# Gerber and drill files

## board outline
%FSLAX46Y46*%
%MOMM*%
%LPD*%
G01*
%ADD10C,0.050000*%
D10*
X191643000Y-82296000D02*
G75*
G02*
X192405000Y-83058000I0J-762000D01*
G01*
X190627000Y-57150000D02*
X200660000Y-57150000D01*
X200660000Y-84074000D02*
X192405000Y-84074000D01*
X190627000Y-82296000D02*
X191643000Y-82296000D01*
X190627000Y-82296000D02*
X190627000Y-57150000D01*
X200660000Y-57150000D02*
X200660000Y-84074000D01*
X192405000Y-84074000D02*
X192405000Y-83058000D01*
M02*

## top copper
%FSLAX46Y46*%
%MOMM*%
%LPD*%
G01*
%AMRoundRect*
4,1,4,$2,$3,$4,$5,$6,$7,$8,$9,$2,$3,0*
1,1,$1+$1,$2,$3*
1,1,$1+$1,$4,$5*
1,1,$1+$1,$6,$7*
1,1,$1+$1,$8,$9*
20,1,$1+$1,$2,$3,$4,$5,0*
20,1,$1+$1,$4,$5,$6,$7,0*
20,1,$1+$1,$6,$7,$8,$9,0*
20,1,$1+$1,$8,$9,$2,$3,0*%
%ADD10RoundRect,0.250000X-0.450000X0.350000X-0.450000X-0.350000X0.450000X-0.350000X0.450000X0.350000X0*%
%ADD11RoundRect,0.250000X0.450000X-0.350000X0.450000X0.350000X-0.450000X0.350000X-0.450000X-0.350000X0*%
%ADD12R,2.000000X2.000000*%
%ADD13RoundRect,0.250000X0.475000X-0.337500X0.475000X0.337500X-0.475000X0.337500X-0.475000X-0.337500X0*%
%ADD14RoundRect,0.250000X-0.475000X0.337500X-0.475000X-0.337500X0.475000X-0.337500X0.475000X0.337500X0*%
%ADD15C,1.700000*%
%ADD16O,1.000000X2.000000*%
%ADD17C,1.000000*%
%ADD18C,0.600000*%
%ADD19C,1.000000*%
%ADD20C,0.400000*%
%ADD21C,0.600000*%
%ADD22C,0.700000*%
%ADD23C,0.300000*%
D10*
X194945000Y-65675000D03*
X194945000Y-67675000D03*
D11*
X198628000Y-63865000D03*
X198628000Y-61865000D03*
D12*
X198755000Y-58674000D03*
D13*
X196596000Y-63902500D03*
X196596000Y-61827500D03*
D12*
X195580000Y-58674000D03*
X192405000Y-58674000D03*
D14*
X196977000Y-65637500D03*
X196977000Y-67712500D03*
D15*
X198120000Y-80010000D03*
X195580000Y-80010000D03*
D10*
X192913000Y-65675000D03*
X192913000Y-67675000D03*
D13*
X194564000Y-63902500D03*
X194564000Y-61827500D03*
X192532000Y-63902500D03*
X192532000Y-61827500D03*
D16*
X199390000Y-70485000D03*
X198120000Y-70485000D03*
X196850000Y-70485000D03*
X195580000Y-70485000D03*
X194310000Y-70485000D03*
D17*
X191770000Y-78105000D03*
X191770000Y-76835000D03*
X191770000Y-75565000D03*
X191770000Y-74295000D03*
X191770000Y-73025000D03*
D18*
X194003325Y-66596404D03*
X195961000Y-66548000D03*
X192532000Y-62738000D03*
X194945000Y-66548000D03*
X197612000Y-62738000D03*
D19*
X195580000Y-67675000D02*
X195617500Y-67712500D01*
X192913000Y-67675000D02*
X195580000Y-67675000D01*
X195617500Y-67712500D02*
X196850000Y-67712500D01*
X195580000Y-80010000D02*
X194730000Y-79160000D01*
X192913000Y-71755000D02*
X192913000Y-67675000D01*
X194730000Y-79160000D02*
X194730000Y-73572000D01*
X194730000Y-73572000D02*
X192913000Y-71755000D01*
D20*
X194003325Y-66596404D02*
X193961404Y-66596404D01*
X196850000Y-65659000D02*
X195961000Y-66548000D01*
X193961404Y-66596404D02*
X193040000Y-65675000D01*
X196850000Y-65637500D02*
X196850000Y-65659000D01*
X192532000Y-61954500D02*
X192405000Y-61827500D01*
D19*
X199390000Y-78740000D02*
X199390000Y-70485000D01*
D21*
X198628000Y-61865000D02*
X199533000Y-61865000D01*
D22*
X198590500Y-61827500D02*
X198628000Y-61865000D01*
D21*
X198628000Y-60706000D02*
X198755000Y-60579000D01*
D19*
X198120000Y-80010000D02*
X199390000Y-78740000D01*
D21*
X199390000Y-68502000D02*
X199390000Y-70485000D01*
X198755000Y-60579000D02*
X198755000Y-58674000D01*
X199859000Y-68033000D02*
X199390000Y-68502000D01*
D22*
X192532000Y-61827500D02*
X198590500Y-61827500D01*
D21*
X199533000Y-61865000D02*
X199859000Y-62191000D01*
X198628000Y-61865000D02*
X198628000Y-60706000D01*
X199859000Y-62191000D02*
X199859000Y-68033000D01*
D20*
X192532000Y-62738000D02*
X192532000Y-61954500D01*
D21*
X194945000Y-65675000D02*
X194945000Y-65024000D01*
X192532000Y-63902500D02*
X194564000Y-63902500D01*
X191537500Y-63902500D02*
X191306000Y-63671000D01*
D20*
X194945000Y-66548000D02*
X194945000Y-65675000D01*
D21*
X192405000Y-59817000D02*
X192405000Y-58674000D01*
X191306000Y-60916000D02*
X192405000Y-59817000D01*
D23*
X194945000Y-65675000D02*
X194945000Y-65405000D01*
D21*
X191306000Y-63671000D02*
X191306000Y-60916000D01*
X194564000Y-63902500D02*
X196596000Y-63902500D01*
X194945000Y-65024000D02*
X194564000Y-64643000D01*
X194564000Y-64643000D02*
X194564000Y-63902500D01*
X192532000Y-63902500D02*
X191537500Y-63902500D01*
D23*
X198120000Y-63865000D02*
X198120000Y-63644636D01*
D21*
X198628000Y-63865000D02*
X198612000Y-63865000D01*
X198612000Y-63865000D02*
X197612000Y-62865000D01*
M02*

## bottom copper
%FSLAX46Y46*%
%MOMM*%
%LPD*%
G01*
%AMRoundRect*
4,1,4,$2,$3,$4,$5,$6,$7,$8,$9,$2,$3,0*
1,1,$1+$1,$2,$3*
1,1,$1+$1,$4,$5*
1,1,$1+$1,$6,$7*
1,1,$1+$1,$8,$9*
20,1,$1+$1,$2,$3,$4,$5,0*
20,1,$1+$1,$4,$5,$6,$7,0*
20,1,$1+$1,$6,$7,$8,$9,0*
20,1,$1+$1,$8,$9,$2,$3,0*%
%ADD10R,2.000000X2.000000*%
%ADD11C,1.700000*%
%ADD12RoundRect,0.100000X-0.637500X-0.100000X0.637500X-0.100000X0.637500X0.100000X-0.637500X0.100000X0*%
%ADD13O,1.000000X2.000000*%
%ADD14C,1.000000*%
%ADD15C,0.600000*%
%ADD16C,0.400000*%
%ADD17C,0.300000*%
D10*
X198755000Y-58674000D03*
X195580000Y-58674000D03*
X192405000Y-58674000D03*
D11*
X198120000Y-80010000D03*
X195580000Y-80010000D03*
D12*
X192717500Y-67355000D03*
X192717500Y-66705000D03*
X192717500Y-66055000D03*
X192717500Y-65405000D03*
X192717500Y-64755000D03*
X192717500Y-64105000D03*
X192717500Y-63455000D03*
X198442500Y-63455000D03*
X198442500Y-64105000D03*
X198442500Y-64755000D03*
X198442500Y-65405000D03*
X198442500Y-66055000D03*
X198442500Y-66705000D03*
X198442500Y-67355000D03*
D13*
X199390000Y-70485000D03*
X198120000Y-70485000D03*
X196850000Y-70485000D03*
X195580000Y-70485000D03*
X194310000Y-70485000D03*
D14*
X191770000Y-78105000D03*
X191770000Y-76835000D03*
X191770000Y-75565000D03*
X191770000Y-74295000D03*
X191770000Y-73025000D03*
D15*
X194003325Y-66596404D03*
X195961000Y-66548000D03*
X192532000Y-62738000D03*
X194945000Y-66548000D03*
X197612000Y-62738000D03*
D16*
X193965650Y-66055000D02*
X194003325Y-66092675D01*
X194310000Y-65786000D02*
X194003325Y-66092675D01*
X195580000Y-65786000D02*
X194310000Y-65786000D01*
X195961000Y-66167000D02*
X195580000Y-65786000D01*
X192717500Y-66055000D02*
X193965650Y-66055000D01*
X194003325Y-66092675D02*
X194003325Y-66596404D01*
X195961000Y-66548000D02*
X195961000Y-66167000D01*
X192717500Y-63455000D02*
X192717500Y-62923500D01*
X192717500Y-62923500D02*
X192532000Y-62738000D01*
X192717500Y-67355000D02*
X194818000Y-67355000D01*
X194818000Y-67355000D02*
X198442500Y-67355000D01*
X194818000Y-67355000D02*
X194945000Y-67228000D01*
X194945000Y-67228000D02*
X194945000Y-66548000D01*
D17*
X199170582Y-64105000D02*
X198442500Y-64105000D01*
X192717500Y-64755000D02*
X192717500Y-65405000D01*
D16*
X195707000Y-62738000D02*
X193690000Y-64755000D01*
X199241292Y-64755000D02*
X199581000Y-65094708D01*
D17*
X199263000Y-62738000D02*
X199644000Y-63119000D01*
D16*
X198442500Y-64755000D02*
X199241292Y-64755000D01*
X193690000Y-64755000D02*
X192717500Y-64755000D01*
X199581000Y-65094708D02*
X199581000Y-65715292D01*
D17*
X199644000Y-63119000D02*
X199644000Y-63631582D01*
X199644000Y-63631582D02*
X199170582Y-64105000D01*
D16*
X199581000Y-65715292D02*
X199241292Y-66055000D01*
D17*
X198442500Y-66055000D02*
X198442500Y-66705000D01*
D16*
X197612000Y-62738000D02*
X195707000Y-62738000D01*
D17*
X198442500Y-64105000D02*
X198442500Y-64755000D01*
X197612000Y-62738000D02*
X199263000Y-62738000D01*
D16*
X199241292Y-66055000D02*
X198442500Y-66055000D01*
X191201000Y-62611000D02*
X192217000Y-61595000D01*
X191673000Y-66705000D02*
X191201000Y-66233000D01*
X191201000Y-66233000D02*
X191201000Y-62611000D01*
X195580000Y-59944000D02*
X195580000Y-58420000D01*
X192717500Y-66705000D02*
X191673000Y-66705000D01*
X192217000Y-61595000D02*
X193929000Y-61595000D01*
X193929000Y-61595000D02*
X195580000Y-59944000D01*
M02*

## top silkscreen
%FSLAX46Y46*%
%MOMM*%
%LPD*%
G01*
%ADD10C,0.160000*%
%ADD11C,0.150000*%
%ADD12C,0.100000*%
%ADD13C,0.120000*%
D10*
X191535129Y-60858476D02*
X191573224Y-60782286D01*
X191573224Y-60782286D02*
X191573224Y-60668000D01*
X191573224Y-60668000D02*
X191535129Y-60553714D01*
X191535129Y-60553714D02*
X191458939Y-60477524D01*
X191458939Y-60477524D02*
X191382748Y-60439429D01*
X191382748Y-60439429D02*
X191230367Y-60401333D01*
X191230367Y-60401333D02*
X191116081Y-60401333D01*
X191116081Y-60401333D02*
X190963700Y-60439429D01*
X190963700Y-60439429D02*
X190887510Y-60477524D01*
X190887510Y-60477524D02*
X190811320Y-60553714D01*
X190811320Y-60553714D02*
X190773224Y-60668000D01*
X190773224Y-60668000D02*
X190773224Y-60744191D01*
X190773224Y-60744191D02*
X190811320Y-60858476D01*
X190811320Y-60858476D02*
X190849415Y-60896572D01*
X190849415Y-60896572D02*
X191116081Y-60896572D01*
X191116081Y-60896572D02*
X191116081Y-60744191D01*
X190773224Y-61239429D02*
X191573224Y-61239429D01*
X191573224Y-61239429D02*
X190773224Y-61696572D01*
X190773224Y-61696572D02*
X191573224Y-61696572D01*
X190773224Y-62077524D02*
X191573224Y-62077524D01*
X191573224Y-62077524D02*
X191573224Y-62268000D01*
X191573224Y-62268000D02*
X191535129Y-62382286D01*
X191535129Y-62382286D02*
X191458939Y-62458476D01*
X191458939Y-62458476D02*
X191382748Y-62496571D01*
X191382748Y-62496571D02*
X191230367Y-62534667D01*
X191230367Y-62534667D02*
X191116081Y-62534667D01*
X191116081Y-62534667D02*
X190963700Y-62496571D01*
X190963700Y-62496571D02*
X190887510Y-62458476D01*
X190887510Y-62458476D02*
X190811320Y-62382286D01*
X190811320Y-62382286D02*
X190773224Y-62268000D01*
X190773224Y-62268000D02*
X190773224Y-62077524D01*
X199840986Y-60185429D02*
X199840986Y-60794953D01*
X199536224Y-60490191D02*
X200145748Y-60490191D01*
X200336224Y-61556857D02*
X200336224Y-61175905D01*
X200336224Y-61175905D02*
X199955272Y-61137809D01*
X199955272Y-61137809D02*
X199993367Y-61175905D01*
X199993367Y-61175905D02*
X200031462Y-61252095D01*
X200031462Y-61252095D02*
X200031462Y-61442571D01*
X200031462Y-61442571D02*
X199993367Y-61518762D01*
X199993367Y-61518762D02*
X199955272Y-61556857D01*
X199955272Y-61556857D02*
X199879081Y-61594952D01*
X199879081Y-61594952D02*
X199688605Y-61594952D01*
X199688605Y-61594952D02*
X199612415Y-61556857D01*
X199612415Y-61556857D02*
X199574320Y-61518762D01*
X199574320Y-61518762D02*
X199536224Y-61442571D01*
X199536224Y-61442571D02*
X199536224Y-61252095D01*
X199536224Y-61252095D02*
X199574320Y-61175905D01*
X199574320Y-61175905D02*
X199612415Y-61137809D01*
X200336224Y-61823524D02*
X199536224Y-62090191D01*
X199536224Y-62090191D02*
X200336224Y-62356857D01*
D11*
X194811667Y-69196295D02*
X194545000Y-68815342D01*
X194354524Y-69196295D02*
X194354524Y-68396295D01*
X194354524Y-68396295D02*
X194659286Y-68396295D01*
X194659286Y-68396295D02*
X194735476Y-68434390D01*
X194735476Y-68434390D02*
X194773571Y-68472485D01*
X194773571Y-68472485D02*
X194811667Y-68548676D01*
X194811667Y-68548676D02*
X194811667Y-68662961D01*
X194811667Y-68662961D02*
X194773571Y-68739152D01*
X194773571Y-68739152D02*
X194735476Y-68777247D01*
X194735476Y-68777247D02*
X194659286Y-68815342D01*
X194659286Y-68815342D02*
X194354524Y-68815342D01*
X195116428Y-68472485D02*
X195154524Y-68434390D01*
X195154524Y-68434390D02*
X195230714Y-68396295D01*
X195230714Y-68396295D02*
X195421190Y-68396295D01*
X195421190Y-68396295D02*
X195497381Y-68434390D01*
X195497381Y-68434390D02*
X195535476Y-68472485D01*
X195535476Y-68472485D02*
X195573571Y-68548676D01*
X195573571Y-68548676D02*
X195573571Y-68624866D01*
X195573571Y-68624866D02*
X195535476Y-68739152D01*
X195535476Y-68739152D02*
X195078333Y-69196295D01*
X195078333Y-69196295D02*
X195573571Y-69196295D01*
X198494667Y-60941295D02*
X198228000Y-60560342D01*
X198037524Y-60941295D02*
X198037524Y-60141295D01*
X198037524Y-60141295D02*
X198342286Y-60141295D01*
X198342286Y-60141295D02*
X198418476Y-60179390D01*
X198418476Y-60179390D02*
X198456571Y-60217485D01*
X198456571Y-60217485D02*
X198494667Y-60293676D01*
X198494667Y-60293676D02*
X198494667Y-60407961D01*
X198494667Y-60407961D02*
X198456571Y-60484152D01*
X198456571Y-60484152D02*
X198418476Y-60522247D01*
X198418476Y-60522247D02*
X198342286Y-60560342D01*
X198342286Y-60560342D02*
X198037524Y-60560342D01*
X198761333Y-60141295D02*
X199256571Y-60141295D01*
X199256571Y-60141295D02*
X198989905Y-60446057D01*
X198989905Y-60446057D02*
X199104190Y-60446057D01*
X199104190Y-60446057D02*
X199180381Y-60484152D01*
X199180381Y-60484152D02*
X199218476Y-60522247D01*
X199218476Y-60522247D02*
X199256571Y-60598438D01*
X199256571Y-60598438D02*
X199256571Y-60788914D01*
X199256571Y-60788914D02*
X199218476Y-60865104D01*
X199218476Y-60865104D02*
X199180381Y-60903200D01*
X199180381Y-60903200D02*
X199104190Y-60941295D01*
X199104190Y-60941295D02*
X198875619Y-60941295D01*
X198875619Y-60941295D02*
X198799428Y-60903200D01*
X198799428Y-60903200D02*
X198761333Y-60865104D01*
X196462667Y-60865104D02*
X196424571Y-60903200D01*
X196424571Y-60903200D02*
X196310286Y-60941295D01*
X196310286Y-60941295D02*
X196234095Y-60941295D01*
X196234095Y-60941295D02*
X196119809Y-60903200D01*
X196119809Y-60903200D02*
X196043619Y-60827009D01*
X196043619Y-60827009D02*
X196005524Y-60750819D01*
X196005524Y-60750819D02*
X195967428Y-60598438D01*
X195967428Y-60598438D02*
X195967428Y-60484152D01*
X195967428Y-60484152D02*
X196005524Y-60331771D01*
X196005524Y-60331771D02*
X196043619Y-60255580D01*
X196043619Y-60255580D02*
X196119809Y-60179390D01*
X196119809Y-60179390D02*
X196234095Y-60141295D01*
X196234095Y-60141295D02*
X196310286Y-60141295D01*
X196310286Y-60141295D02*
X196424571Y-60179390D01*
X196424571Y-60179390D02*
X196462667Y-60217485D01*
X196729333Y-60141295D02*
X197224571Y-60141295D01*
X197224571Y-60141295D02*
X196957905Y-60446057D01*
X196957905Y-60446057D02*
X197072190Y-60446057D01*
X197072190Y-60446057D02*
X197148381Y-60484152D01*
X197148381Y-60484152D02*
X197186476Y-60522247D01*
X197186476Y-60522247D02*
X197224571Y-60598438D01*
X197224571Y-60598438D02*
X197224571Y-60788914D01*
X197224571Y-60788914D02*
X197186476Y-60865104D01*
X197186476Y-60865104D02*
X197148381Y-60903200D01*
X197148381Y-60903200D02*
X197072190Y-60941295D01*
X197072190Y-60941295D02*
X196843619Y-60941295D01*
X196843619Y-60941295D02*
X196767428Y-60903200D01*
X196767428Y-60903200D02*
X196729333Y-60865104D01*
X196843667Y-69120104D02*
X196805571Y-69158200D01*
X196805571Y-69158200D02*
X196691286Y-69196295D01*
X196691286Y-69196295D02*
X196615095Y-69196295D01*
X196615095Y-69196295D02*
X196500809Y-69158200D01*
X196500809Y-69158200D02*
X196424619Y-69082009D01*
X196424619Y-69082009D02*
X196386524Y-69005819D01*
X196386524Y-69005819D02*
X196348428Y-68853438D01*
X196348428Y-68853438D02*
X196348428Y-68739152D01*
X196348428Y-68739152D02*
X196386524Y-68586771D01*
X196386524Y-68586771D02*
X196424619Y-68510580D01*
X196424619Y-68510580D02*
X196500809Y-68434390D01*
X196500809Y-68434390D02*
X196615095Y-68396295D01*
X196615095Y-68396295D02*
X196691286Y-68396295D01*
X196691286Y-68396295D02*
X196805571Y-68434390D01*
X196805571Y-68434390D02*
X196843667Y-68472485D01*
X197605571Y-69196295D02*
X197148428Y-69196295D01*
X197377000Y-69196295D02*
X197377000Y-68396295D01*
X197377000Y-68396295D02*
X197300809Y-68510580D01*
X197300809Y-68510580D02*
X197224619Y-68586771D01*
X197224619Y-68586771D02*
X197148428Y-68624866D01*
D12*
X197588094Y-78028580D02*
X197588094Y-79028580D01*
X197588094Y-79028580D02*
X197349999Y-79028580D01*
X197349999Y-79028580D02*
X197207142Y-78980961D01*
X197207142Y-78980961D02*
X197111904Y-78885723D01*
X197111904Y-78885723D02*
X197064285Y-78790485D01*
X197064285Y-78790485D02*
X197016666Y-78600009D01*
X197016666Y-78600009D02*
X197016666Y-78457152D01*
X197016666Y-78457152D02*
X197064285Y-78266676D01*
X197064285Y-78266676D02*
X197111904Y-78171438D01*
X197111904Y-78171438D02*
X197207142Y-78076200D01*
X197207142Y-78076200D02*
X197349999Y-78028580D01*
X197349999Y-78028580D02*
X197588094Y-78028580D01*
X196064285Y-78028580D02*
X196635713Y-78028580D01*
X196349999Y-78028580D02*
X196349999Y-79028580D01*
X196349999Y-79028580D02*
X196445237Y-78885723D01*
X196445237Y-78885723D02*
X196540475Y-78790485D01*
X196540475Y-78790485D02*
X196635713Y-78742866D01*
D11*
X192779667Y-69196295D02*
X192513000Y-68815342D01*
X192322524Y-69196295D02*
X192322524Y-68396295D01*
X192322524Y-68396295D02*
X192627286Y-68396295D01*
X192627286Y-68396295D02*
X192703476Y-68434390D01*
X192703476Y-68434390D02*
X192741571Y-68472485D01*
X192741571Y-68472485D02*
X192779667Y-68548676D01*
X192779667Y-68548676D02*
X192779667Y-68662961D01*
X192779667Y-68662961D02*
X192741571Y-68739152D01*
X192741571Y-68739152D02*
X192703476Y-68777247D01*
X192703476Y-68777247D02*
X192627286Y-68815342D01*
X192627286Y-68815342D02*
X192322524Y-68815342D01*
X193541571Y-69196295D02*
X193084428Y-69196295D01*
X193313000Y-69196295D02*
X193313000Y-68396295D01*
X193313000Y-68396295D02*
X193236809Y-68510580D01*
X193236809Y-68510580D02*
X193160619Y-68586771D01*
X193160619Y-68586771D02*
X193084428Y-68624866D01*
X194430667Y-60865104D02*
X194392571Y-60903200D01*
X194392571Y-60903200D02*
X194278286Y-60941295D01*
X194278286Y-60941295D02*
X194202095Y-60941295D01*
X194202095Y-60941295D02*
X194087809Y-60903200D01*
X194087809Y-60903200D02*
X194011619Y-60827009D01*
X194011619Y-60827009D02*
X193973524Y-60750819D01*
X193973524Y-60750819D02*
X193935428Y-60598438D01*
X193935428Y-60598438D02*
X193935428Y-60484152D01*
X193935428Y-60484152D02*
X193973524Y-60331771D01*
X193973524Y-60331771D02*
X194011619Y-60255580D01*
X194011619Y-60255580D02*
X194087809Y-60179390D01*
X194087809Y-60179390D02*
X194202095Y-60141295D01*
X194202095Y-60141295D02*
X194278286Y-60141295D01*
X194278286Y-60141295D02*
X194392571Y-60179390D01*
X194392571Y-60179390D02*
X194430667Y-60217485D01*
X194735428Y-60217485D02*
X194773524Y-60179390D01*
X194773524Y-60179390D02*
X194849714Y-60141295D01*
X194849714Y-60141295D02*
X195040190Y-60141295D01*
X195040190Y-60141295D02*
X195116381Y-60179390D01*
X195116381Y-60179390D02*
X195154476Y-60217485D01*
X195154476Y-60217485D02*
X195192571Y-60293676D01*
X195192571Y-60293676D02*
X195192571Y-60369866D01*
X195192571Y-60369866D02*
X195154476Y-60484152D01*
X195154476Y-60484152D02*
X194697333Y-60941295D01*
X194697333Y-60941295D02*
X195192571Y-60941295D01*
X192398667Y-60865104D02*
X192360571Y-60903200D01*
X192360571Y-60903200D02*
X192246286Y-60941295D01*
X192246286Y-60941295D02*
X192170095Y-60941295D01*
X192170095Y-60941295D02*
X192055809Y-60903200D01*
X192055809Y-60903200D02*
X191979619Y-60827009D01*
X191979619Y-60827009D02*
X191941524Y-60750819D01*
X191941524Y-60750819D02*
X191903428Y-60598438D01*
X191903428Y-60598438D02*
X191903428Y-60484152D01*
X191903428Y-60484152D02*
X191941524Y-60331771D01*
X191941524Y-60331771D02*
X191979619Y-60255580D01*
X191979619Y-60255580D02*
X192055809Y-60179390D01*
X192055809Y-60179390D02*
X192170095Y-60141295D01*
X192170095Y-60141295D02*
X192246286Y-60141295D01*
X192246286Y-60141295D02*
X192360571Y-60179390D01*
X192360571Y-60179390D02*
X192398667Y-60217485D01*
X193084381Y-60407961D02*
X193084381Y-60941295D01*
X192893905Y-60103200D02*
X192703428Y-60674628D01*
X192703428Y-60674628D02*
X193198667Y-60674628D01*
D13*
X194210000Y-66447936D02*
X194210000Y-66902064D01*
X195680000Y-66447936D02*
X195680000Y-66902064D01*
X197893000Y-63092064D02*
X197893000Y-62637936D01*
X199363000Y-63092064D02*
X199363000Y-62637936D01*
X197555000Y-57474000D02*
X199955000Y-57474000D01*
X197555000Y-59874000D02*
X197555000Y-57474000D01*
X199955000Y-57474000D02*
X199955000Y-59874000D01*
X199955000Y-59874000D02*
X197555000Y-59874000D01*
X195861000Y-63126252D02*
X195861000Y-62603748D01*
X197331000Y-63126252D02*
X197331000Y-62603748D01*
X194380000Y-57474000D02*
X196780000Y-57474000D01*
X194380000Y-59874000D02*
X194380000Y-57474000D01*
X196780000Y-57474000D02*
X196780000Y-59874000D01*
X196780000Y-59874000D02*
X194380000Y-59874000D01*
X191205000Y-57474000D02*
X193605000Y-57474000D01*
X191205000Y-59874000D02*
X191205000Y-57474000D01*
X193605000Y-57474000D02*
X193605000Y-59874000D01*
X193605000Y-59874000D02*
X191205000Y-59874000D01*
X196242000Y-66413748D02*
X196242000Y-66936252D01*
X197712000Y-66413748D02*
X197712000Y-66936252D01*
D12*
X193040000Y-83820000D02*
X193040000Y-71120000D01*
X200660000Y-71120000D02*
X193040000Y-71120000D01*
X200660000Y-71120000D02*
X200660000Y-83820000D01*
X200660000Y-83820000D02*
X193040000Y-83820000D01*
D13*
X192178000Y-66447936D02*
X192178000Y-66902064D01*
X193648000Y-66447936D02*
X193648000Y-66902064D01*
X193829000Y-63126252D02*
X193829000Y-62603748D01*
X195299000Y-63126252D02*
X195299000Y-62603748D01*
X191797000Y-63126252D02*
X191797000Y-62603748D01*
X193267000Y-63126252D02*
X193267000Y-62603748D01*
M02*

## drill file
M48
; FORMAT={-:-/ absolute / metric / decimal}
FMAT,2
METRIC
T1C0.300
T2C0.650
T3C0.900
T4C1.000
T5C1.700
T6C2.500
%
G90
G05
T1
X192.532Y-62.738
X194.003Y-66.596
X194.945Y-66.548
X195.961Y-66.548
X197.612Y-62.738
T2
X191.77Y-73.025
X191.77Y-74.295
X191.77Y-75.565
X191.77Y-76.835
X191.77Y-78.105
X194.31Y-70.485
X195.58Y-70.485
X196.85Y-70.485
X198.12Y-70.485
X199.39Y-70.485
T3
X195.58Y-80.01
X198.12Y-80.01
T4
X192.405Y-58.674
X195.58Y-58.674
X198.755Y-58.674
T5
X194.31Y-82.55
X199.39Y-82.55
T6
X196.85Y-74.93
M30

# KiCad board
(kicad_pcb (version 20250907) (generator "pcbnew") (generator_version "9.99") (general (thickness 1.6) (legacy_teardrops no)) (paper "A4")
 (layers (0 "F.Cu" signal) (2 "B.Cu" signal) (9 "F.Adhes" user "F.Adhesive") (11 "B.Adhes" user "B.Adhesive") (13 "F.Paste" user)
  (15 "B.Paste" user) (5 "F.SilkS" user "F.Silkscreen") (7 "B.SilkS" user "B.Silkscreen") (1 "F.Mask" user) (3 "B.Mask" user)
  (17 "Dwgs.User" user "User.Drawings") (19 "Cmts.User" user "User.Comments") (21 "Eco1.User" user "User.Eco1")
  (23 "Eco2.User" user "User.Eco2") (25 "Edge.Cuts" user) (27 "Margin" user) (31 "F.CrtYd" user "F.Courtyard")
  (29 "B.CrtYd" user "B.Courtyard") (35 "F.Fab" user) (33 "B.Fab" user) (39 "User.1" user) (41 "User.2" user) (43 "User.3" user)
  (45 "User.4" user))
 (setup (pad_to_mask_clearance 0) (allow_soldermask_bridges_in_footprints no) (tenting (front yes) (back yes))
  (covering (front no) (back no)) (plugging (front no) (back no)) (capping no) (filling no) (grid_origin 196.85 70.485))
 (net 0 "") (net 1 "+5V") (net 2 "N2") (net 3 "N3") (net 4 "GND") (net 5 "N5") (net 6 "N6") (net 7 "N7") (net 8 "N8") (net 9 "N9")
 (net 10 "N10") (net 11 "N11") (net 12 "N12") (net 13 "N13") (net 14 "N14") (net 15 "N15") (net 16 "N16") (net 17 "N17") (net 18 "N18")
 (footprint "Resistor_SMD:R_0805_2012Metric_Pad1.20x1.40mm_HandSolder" (layer "F.Cu") (at 194.945 66.675 -90)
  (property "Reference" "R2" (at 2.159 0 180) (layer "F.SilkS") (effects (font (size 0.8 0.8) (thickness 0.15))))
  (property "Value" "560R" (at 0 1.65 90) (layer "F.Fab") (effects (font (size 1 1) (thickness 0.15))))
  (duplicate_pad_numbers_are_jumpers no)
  (fp_line (start -0.227064 0.735) (end 0.227064 0.735) (stroke (width 0.12) (type solid)) (layer "F.SilkS"))
  (fp_line (start -0.227064 -0.735) (end 0.227064 -0.735) (stroke (width 0.12) (type solid)) (layer "F.SilkS"))
  (pad "1" smd roundrect (at -1 0 270) (size 1.2 1.4) (layers "F.Cu" "F.Mask" "F.Paste") (roundrect_rratio 0.208333) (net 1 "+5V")
   (tenting (front none) (back none)))
  (pad "2" smd roundrect (at 1 0 270) (size 1.2 1.4) (layers "F.Cu" "F.Mask" "F.Paste") (roundrect_rratio 0.208333) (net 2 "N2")
   (tenting (front none) (back none))))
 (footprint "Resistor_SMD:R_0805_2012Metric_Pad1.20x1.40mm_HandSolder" (layer "F.Cu") (at 198.628 62.865 90)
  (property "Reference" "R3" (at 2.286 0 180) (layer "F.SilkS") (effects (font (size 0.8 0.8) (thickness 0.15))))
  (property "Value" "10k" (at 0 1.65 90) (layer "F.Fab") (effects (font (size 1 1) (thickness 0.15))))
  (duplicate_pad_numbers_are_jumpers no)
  (fp_line (start -0.227064 -0.735) (end 0.227064 -0.735) (stroke (width 0.12) (type solid)) (layer "F.SilkS"))
  (fp_line (start -0.227064 0.735) (end 0.227064 0.735) (stroke (width 0.12) (type solid)) (layer "F.SilkS"))
  (pad "1" smd roundrect (at -1 0 90) (size 1.2 1.4) (layers "F.Cu" "F.Mask" "F.Paste") (roundrect_rratio 0.208333) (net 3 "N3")
   (tenting (front none) (back none)))
  (pad "2" smd roundrect (at 1 0 90) (size 1.2 1.4) (layers "F.Cu" "F.Mask" "F.Paste") (roundrect_rratio 0.208333) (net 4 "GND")
   (tenting (front none) (back none))))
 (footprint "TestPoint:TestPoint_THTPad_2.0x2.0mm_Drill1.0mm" (layer "F.Cu") (at 198.755 58.674 180)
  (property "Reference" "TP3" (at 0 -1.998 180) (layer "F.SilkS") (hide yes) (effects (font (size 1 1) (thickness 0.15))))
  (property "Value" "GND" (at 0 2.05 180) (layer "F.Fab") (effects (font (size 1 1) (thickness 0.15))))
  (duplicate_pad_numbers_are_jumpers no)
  (fp_line (start 1.2 1.2) (end -1.2 1.2) (stroke (width 0.12) (type solid)) (layer "F.SilkS"))
  (fp_line (start 1.2 -1.2) (end 1.2 1.2) (stroke (width 0.12) (type solid)) (layer "F.SilkS"))
  (fp_line (start -1.2 1.2) (end -1.2 -1.2) (stroke (width 0.12) (type solid)) (layer "F.SilkS"))
  (fp_line (start -1.2 -1.2) (end 1.2 -1.2) (stroke (width 0.12) (type solid)) (layer "F.SilkS"))
  (pad "1" thru_hole rect (at 0 0 180) (size 2 2) (drill 1) (layers "*.Cu" "*.Mask") (remove_unused_layers no) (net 4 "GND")
   (tenting (front none) (back none))))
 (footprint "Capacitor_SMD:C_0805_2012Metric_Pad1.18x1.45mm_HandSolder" (layer "F.Cu") (at 196.596 62.865 90)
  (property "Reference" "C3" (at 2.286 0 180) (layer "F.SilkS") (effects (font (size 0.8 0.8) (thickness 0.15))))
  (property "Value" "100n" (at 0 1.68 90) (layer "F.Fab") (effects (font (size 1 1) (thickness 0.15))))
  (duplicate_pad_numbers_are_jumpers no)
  (fp_line (start -0.261252 -0.735) (end 0.261252 -0.735) (stroke (width 0.12) (type solid)) (layer "F.SilkS"))
  (fp_line (start -0.261252 0.735) (end 0.261252 0.735) (stroke (width 0.12) (type solid)) (layer "F.SilkS"))
  (pad "1" smd roundrect (at -1.0375 0 90) (size 1.175 1.45) (layers "F.Cu" "F.Mask" "F.Paste") (roundrect_rratio 0.212766) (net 1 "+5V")
   (tenting (front none) (back none)))
  (pad "2" smd roundrect (at 1.0375 0 90) (size 1.175 1.45) (layers "F.Cu" "F.Mask" "F.Paste") (roundrect_rratio 0.212766) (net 4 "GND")
   (tenting (front none) (back none))))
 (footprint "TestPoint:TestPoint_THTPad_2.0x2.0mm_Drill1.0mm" (layer "F.Cu") (at 195.58 58.674 180)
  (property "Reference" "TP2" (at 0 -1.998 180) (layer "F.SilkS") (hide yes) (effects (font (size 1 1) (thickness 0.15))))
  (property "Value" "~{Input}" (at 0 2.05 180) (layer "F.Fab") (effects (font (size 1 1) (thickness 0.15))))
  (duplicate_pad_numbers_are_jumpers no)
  (fp_line (start 1.2 1.2) (end -1.2 1.2) (stroke (width 0.12) (type solid)) (layer "F.SilkS"))
  (fp_line (start 1.2 -1.2) (end 1.2 1.2) (stroke (width 0.12) (type solid)) (layer "F.SilkS"))
  (fp_line (start -1.2 1.2) (end -1.2 -1.2) (stroke (width 0.12) (type solid)) (layer "F.SilkS"))
  (fp_line (start -1.2 -1.2) (end 1.2 -1.2) (stroke (width 0.12) (type solid)) (layer "F.SilkS"))
  (pad "1" thru_hole rect (at 0 0 180) (size 2 2) (drill 1) (layers "*.Cu" "*.Mask") (remove_unused_layers no) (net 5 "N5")
   (tenting (front none) (back none))))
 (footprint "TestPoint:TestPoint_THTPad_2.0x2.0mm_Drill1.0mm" (layer "F.Cu") (at 192.405 58.674 180)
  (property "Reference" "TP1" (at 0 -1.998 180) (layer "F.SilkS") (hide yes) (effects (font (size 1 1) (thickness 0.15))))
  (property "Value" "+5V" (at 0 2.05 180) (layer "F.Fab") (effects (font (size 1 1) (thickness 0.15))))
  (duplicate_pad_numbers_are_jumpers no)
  (fp_line (start 1.2 1.2) (end -1.2 1.2) (stroke (width 0.12) (type solid)) (layer "F.SilkS"))
  (fp_line (start 1.2 -1.2) (end 1.2 1.2) (stroke (width 0.12) (type solid)) (layer "F.SilkS"))
  (fp_line (start -1.2 1.2) (end -1.2 -1.2) (stroke (width 0.12) (type solid)) (layer "F.SilkS"))
  (fp_line (start -1.2 -1.2) (end 1.2 -1.2) (stroke (width 0.12) (type solid)) (layer "F.SilkS"))
  (pad "1" thru_hole rect (at 0 0 180) (size 2 2) (drill 1) (layers "*.Cu" "*.Mask") (remove_unused_layers no) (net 1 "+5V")
   (tenting (front none) (back none))))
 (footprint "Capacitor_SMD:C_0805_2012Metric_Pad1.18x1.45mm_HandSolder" (layer "F.Cu") (at 196.977 66.675 -90)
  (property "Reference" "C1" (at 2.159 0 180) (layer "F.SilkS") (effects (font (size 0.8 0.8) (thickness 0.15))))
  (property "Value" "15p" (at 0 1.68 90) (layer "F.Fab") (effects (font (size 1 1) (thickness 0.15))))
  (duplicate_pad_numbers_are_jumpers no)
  (fp_line (start -0.261252 0.735) (end 0.261252 0.735) (stroke (width 0.12) (type solid)) (layer "F.SilkS"))
  (fp_line (start -0.261252 -0.735) (end 0.261252 -0.735) (stroke (width 0.12) (type solid)) (layer "F.SilkS"))
  (pad "1" smd roundrect (at -1.0375 0 270) (size 1.175 1.45) (layers "F.Cu" "F.Mask" "F.Paste") (roundrect_rratio 0.212766) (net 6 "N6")
   (tenting (front none) (back none)))
  (pad "2" smd roundrect (at 1.0375 0 270) (size 1.175 1.45) (layers "F.Cu" "F.Mask" "F.Paste") (roundrect_rratio 0.212766) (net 2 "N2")
   (tenting (front none) (back none))))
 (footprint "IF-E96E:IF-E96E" (layer "F.Cu") (at 196.85 80.01 180)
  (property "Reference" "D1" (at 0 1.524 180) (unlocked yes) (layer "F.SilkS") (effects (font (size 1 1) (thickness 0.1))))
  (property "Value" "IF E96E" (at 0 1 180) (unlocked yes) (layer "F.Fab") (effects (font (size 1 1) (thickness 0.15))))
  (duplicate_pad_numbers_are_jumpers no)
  (fp_line (start 3.81 -3.81) (end 3.81 8.89) (stroke (width 0.1) (type default)) (layer "F.SilkS"))
  (fp_line (start -3.81 8.89) (end 3.81 8.89) (stroke (width 0.1) (type default)) (layer "F.SilkS"))
  (fp_line (start -3.81 8.89) (end -3.81 -3.81) (stroke (width 0.1) (type default)) (layer "F.SilkS"))
  (fp_line (start -3.81 -3.81) (end 3.81 -3.81) (stroke (width 0.1) (type default)) (layer "F.SilkS"))
  (pad "" np_thru_hole circle (at -2.54 -2.54 180) (size 1.7 1.7) (drill 1.7) (layers "*.Cu" "*.Mask") (tenting (front none) (back none)))
  (pad "" np_thru_hole circle (at 0 5.08 180) (size 2.5 2.5) (drill 2.5) (layers "*.Cu" "*.Mask") (tenting (front none) (back none)))
  (pad "" np_thru_hole circle (at 2.54 -2.54 180) (size 1.7 1.7) (drill 1.7) (layers "*.Cu" "*.Mask") (tenting (front none) (back none)))
  (pad "1" thru_hole circle (at -1.27 0 180) (size 1.7 1.7) (drill 0.9) (layers "*.Cu" "*.Mask") (remove_unused_layers no) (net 4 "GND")
   (tenting (front none) (back none)))
  (pad "2" thru_hole circle (at 1.27 0 180) (size 1.7 1.7) (drill 0.9) (layers "*.Cu" "*.Mask") (remove_unused_layers no) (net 2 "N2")
   (tenting (front none) (back none))))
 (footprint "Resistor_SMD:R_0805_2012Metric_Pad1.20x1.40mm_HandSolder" (layer "F.Cu") (at 192.913 66.675 -90)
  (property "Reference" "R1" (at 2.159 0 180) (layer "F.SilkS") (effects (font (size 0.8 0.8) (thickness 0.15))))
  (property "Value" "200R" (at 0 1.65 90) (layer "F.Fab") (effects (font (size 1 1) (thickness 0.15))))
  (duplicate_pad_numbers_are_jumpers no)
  (fp_line (start -0.227064 0.735) (end 0.227064 0.735) (stroke (width 0.12) (type solid)) (layer "F.SilkS"))
  (fp_line (start -0.227064 -0.735) (end 0.227064 -0.735) (stroke (width 0.12) (type solid)) (layer "F.SilkS"))
  (pad "1" smd roundrect (at -1 0 270) (size 1.2 1.4) (layers "F.Cu" "F.Mask" "F.Paste") (roundrect_rratio 0.208333) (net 6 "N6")
   (tenting (front none) (back none)))
  (pad "2" smd roundrect (at 1 0 270) (size 1.2 1.4) (layers "F.Cu" "F.Mask" "F.Paste") (roundrect_rratio 0.208333) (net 2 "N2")
   (tenting (front none) (back none))))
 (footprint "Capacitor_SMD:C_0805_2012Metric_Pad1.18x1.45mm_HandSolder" (layer "F.Cu") (at 194.564 62.865 90)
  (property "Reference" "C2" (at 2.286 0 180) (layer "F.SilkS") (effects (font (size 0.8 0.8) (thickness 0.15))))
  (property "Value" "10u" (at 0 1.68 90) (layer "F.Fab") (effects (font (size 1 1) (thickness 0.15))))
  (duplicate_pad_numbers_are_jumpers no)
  (fp_line (start -0.261252 -0.735) (end 0.261252 -0.735) (stroke (width 0.12) (type solid)) (layer "F.SilkS"))
  (fp_line (start -0.261252 0.735) (end 0.261252 0.735) (stroke (width 0.12) (type solid)) (layer "F.SilkS"))
  (pad "1" smd roundrect (at -1.0375 0 90) (size 1.175 1.45) (layers "F.Cu" "F.Mask" "F.Paste") (roundrect_rratio 0.212766) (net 1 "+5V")
   (tenting (front none) (back none)))
  (pad "2" smd roundrect (at 1.0375 0 90) (size 1.175 1.45) (layers "F.Cu" "F.Mask" "F.Paste") (roundrect_rratio 0.212766) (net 4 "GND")
   (tenting (front none) (back none))))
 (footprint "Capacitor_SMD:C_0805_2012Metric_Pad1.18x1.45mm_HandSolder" (layer "F.Cu") (at 192.532 62.865 90)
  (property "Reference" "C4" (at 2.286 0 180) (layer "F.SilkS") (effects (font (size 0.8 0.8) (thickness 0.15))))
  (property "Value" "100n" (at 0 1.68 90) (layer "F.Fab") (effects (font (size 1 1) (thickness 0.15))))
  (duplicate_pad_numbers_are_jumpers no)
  (fp_line (start -0.261252 -0.735) (end 0.261252 -0.735) (stroke (width 0.12) (type solid)) (layer "F.SilkS"))
  (fp_line (start -0.261252 0.735) (end 0.261252 0.735) (stroke (width 0.12) (type solid)) (layer "F.SilkS"))
  (pad "1" smd roundrect (at -1.0375 0 90) (size 1.175 1.45) (layers "F.Cu" "F.Mask" "F.Paste") (roundrect_rratio 0.212766) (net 1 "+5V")
   (tenting (front none) (back none)))
  (pad "2" smd roundrect (at 1.0375 0 90) (size 1.175 1.45) (layers "F.Cu" "F.Mask" "F.Paste") (roundrect_rratio 0.212766) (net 4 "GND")
   (tenting (front none) (back none))))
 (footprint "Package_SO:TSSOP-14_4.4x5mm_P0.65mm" (layer "B.Cu") (at 195.58 65.405)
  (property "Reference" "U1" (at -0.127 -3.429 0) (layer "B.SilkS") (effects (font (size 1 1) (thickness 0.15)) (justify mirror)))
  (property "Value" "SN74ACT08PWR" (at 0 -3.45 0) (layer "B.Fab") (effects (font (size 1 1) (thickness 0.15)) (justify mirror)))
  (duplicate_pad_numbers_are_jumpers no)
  (pad "1" smd roundrect (at -2.8625 1.95) (size 1.475 0.4) (layers "B.Cu" "B.Mask" "B.Paste") (roundrect_rratio 0.25) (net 1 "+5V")
   (tenting (front none) (back none)))
  (pad "2" smd roundrect (at -2.8625 1.3) (size 1.475 0.4) (layers "B.Cu" "B.Mask" "B.Paste") (roundrect_rratio 0.25) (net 5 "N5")
   (tenting (front none) (back none)))
  (pad "3" smd roundrect (at -2.8625 0.65) (size 1.475 0.4) (layers "B.Cu" "B.Mask" "B.Paste") (roundrect_rratio 0.25) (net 6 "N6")
   (tenting (front none) (back none)))
  (pad "4" smd roundrect (at -2.8625 0) (size 1.475 0.4) (layers "B.Cu" "B.Mask" "B.Paste") (roundrect_rratio 0.25) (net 3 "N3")
   (tenting (front none) (back none)))
  (pad "5" smd roundrect (at -2.8625 -0.65) (size 1.475 0.4) (layers "B.Cu" "B.Mask" "B.Paste") (roundrect_rratio 0.25) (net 3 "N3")
   (tenting (front none) (back none)))
  (pad "6" smd roundrect (at -2.8625 -1.3) (size 1.475 0.4) (layers "B.Cu" "B.Mask" "B.Paste") (roundrect_rratio 0.25) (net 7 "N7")
   (tenting (front none) (back none)))
  (pad "7" smd roundrect (at -2.8625 -1.95) (size 1.475 0.4) (layers "B.Cu" "B.Mask" "B.Paste") (roundrect_rratio 0.25) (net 4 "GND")
   (tenting (front none) (back none)))
  (pad "8" smd roundrect (at 2.8625 -1.95) (size 1.475 0.4) (layers "B.Cu" "B.Mask" "B.Paste") (roundrect_rratio 0.25) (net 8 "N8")
   (tenting (front none) (back none)))
  (pad "9" smd roundrect (at 2.8625 -1.3) (size 1.475 0.4) (layers "B.Cu" "B.Mask" "B.Paste") (roundrect_rratio 0.25) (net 3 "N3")
   (tenting (front none) (back none)))
  (pad "10" smd roundrect (at 2.8625 -0.65) (size 1.475 0.4) (layers "B.Cu" "B.Mask" "B.Paste") (roundrect_rratio 0.25) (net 3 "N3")
   (tenting (front none) (back none)))
  (pad "11" smd roundrect (at 2.8625 0) (size 1.475 0.4) (layers "B.Cu" "B.Mask" "B.Paste") (roundrect_rratio 0.25) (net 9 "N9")
   (tenting (front none) (back none)))
  (pad "12" smd roundrect (at 2.8625 0.65) (size 1.475 0.4) (layers "B.Cu" "B.Mask" "B.Paste") (roundrect_rratio 0.25) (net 3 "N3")
   (tenting (front none) (back none)))
  (pad "13" smd roundrect (at 2.8625 1.3) (size 1.475 0.4) (layers "B.Cu" "B.Mask" "B.Paste") (roundrect_rratio 0.25) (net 3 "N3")
   (tenting (front none) (back none)))
  (pad "14" smd roundrect (at 2.8625 1.95) (size 1.475 0.4) (layers "B.Cu" "B.Mask" "B.Paste") (roundrect_rratio 0.25) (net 1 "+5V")
   (tenting (front none) (back none))))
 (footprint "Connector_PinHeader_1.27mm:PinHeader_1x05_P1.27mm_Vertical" (layer "B.Cu") (at 199.39 70.485 90)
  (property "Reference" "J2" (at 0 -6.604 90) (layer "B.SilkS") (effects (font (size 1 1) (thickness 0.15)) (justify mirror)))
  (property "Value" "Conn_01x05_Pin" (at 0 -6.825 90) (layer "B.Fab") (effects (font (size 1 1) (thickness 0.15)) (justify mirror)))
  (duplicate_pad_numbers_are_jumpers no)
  (pad "1" thru_hole oval (at 0 0 90) (size 2 1) (drill 0.65) (layers "*.Cu" "*.Mask") (remove_unused_layers no) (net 4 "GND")
   (tenting (front none) (back none)))
  (pad "2" thru_hole oval (at 0 -1.27 90) (size 2 1) (drill 0.65) (layers "*.Cu" "*.Mask") (remove_unused_layers no) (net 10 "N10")
   (thermal_bridge_angle 45) (tenting (front none) (back none)))
  (pad "3" thru_hole oval (at 0 -2.54 90) (size 2 1) (drill 0.65) (layers "*.Cu" "*.Mask") (remove_unused_layers no) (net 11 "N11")
   (thermal_bridge_angle 45) (tenting (front none) (back none)))
  (pad "4" thru_hole oval (at 0 -3.81 90) (size 2 1) (drill 0.65) (layers "*.Cu" "*.Mask") (remove_unused_layers no) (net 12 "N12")
   (thermal_bridge_angle 45) (tenting (front none) (back none)))
  (pad "5" thru_hole oval (at 0 -5.08 90) (size 2 1) (drill 0.65) (layers "*.Cu" "*.Mask") (remove_unused_layers no) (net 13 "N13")
   (thermal_bridge_angle 45) (tenting (front none) (back none))))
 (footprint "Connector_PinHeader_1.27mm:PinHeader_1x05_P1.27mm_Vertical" (layer "B.Cu") (at 191.77 78.105)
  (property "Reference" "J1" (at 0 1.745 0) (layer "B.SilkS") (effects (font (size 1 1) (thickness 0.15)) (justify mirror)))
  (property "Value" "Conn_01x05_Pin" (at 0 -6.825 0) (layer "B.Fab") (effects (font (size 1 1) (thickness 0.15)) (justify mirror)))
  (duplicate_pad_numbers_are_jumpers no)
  (pad "1" thru_hole circle (at 0 0) (size 1 1) (drill 0.65) (layers "*.Cu" "*.Mask") (remove_unused_layers no) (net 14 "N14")
   (thermal_bridge_angle 90) (tenting (front none) (back none)))
  (pad "2" thru_hole circle (at 0 -1.27) (size 1 1) (drill 0.65) (layers "*.Cu" "*.Mask") (remove_unused_layers no) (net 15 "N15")
   (tenting (front none) (back none)))
  (pad "3" thru_hole circle (at 0 -2.54) (size 1 1) (drill 0.65) (layers "*.Cu" "*.Mask") (remove_unused_layers no) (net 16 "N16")
   (tenting (front none) (back none)))
  (pad "4" thru_hole circle (at 0 -3.81) (size 1 1) (drill 0.65) (layers "*.Cu" "*.Mask") (remove_unused_layers no) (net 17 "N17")
   (tenting (front none) (back none)))
  (pad "5" thru_hole circle (at 0 -5.08) (size 1 1) (drill 0.65) (layers "*.Cu" "*.Mask") (remove_unused_layers no) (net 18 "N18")
   (thermal_bridge_angle 90) (tenting (front none) (back none))))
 (gr_arc (start 191.643 82.296) (mid 192.181815 82.519185) (end 192.405 83.058) (stroke (width 0.05) (type default)) (layer "Edge.Cuts"))
 (gr_line (start 190.627 57.15) (end 200.66 57.15) (stroke (width 0.05) (type default)) (layer "Edge.Cuts"))
 (gr_line (start 200.66 84.074) (end 192.405 84.074) (stroke (width 0.05) (type default)) (layer "Edge.Cuts"))
 (gr_line (start 190.627 82.296) (end 191.643 82.296) (stroke (width 0.05) (type default)) (layer "Edge.Cuts"))
 (gr_line (start 190.627 82.296) (end 190.627 57.15) (stroke (width 0.05) (type default)) (layer "Edge.Cuts"))
 (gr_line (start 200.66 57.15) (end 200.66 84.074) (stroke (width 0.05) (type default)) (layer "Edge.Cuts"))
 (gr_line (start 192.405 84.074) (end 192.405 83.058) (stroke (width 0.05) (type solid)) (layer "Edge.Cuts"))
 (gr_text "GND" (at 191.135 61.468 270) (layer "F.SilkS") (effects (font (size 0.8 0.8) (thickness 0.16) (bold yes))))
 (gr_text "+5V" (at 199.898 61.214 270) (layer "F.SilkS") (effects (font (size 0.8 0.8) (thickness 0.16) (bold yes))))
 (segment (start 195.58 67.675) (end 195.6175 67.7125) (width 1) (layer "F.Cu") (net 2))
 (segment (start 192.913 67.675) (end 195.58 67.675) (width 1) (layer "F.Cu") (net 2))
 (segment (start 195.6175 67.7125) (end 196.85 67.7125) (width 1) (layer "F.Cu") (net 2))
 (segment (start 195.58 80.01) (end 194.73 79.16) (width 1) (layer "F.Cu") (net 2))
 (segment (start 192.913 71.755) (end 192.913 67.675) (width 1) (layer "F.Cu") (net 2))
 (segment (start 194.73 79.16) (end 194.73 73.572) (width 1) (layer "F.Cu") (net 2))
 (segment (start 194.73 73.572) (end 192.913 71.755) (width 1) (layer "F.Cu") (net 2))
 (segment (start 194.003325 66.596404) (end 193.961404 66.596404) (width 0.4) (layer "F.Cu") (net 6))
 (segment (start 196.85 65.659) (end 195.961 66.548) (width 0.4) (layer "F.Cu") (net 6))
 (segment (start 193.961404 66.596404) (end 193.04 65.675) (width 0.4) (layer "F.Cu") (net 6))
 (segment (start 196.85 65.6375) (end 196.85 65.659) (width 0.4) (layer "F.Cu") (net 6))
 (via (at 194.003325 66.596404) (size 0.6) (drill 0.3) (layers "F.Cu" "B.Cu") (tenting (front none) (back none)) (capping none)
  (covering (front none) (back none)) (plugging (front none) (back none)) (filling none) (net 6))
 (via (at 195.961 66.548) (size 0.6) (drill 0.3) (layers "F.Cu" "B.Cu") (tenting (front none) (back none)) (capping none)
  (covering (front none) (back none)) (plugging (front none) (back none)) (filling none) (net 6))
 (segment (start 193.96565 66.055) (end 194.003325 66.092675) (width 0.4) (layer "B.Cu") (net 6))
 (segment (start 194.31 65.786) (end 194.003325 66.092675) (width 0.4) (layer "B.Cu") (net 6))
 (segment (start 195.58 65.786) (end 194.31 65.786) (width 0.4) (layer "B.Cu") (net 6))
 (segment (start 195.961 66.167) (end 195.58 65.786) (width 0.4) (layer "B.Cu") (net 6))
 (segment (start 192.7175 66.055) (end 193.96565 66.055) (width 0.4) (layer "B.Cu") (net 6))
 (segment (start 194.003325 66.092675) (end 194.003325 66.596404) (width 0.4) (layer "B.Cu") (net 6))
 (segment (start 195.961 66.548) (end 195.961 66.167) (width 0.4) (layer "B.Cu") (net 6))
 (segment (start 192.532 61.9545) (end 192.405 61.8275) (width 0.4) (layer "F.Cu") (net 4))
 (segment (start 199.39 78.74) (end 199.39 70.485) (width 1) (layer "F.Cu") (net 4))
 (segment (start 198.628 61.865) (end 199.533 61.865) (width 0.6) (layer "F.Cu") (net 4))
 (segment (start 198.5905 61.8275) (end 198.628 61.865) (width 0.7) (layer "F.Cu") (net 4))
 (segment (start 198.628 60.706) (end 198.755 60.579) (width 0.6) (layer "F.Cu") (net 4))
 (segment (start 198.12 80.01) (end 199.39 78.74) (width 1) (layer "F.Cu") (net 4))
 (segment (start 199.39 68.502) (end 199.39 70.485) (width 0.6) (layer "F.Cu") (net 4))
 (segment (start 198.755 60.579) (end 198.755 58.674) (width 0.6) (layer "F.Cu") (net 4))
 (segment (start 199.859 68.033) (end 199.39 68.502) (width 0.6) (layer "F.Cu") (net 4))
 (segment (start 192.532 61.8275) (end 198.5905 61.8275) (width 0.7) (layer "F.Cu") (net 4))
 (segment (start 199.533 61.865) (end 199.859 62.191) (width 0.6) (layer "F.Cu") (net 4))
 (segment (start 198.628 61.865) (end 198.628 60.706) (width 0.6) (layer "F.Cu") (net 4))
 (segment (start 199.859 62.191) (end 199.859 68.033) (width 0.6) (layer "F.Cu") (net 4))
 (segment (start 192.532 62.738) (end 192.532 61.9545) (width 0.4) (layer "F.Cu") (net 4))
 (via (at 192.532 62.738) (size 0.6) (drill 0.3) (layers "F.Cu" "B.Cu") (tenting (front none) (back none)) (capping none)
  (covering (front none) (back none)) (plugging (front none) (back none)) (filling none) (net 4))
 (segment (start 192.7175 63.455) (end 192.7175 62.9235) (width 0.4) (layer "B.Cu") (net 4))
 (segment (start 192.7175 62.9235) (end 192.532 62.738) (width 0.4) (layer "B.Cu") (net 4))
 (segment (start 194.945 65.675) (end 194.945 65.024) (width 0.6) (layer "F.Cu") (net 1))
 (segment (start 192.532 63.9025) (end 194.564 63.9025) (width 0.6) (layer "F.Cu") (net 1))
 (segment (start 191.5375 63.9025) (end 191.306 63.671) (width 0.6) (layer "F.Cu") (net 1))
 (segment (start 194.945 66.548) (end 194.945 65.675) (width 0.4) (layer "F.Cu") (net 1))
 (segment (start 192.405 59.817) (end 192.405 58.674) (width 0.6) (layer "F.Cu") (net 1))
 (segment (start 191.306 60.916) (end 192.405 59.817) (width 0.6) (layer "F.Cu") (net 1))
 (segment (start 194.945 65.675) (end 194.945 65.405) (width 0.3) (layer "F.Cu") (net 1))
 (segment (start 191.306 63.671) (end 191.306 60.916) (width 0.6) (layer "F.Cu") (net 1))
 (segment (start 194.564 63.9025) (end 196.596 63.9025) (width 0.6) (layer "F.Cu") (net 1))
 (segment (start 194.945 65.024) (end 194.564 64.643) (width 0.6) (layer "F.Cu") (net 1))
 (segment (start 194.564 64.643) (end 194.564 63.9025) (width 0.6) (layer "F.Cu") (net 1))
 (segment (start 192.532 63.9025) (end 191.5375 63.9025) (width 0.6) (layer "F.Cu") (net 1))
 (via (at 194.945 66.548) (size 0.6) (drill 0.3) (layers "F.Cu" "B.Cu") (tenting (front none) (back none)) (capping none)
  (covering (front none) (back none)) (plugging (front none) (back none)) (filling none) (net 1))
 (segment (start 192.7175 67.355) (end 194.818 67.355) (width 0.4) (layer "B.Cu") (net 1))
 (segment (start 194.818 67.355) (end 198.4425 67.355) (width 0.4) (layer "B.Cu") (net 1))
 (segment (start 194.818 67.355) (end 194.945 67.228) (width 0.4) (layer "B.Cu") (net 1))
 (segment (start 194.945 67.228) (end 194.945 66.548) (width 0.4) (layer "B.Cu") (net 1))
 (segment (start 198.12 63.865) (end 198.12 63.644636) (width 0.3) (layer "F.Cu") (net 3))
 (segment (start 198.628 63.865) (end 198.612 63.865) (width 0.6) (layer "F.Cu") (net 3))
 (segment (start 198.612 63.865) (end 197.612 62.865) (width 0.6) (layer "F.Cu") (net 3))
 (via (at 197.612 62.738) (size 0.6) (drill 0.3) (layers "F.Cu" "B.Cu") (tenting (front none) (back none)) (capping none)
  (covering (front none) (back none)) (plugging (front none) (back none)) (filling none) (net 3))
 (segment (start 199.170582 64.105) (end 198.4425 64.105) (width 0.3) (layer "B.Cu") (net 3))
 (segment (start 192.7175 64.755) (end 192.7175 65.405) (width 0.3) (layer "B.Cu") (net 3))
 (segment (start 195.707 62.738) (end 193.69 64.755) (width 0.4) (layer "B.Cu") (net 3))
 (segment (start 199.241292 64.755) (end 199.581 65.094708) (width 0.4) (layer "B.Cu") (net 3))
 (segment (start 199.263 62.738) (end 199.644 63.119) (width 0.3) (layer "B.Cu") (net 3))
 (segment (start 198.4425 64.755) (end 199.241292 64.755) (width 0.4) (layer "B.Cu") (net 3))
 (segment (start 193.69 64.755) (end 192.7175 64.755) (width 0.4) (layer "B.Cu") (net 3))
 (segment (start 199.581 65.094708) (end 199.581 65.715292) (width 0.4) (layer "B.Cu") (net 3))
 (segment (start 199.644 63.119) (end 199.644 63.631582) (width 0.3) (layer "B.Cu") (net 3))
 (segment (start 199.644 63.631582) (end 199.170582 64.105) (width 0.3) (layer "B.Cu") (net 3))
 (segment (start 199.581 65.715292) (end 199.241292 66.055) (width 0.4) (layer "B.Cu") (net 3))
 (segment (start 198.4425 66.055) (end 198.4425 66.705) (width 0.3) (layer "B.Cu") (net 3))
 (segment (start 197.612 62.738) (end 195.707 62.738) (width 0.4) (layer "B.Cu") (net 3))
 (segment (start 198.4425 64.105) (end 198.4425 64.755) (width 0.3) (layer "B.Cu") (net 3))
 (segment (start 197.612 62.738) (end 199.263 62.738) (width 0.3) (layer "B.Cu") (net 3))
 (segment (start 199.241292 66.055) (end 198.4425 66.055) (width 0.4) (layer "B.Cu") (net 3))
 (segment (start 191.201 62.611) (end 192.217 61.595) (width 0.4) (layer "B.Cu") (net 5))
 (segment (start 191.673 66.705) (end 191.201 66.233) (width 0.4) (layer "B.Cu") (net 5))
 (segment (start 191.201 66.233) (end 191.201 62.611) (width 0.4) (layer "B.Cu") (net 5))
 (segment (start 195.58 59.944) (end 195.58 58.42) (width 0.4) (layer "B.Cu") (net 5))
 (segment (start 192.7175 66.705) (end 191.673 66.705) (width 0.4) (layer "B.Cu") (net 5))
 (segment (start 192.217 61.595) (end 193.929 61.595) (width 0.4) (layer "B.Cu") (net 5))
 (segment (start 193.929 61.595) (end 195.58 59.944) (width 0.4) (layer "B.Cu") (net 5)))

